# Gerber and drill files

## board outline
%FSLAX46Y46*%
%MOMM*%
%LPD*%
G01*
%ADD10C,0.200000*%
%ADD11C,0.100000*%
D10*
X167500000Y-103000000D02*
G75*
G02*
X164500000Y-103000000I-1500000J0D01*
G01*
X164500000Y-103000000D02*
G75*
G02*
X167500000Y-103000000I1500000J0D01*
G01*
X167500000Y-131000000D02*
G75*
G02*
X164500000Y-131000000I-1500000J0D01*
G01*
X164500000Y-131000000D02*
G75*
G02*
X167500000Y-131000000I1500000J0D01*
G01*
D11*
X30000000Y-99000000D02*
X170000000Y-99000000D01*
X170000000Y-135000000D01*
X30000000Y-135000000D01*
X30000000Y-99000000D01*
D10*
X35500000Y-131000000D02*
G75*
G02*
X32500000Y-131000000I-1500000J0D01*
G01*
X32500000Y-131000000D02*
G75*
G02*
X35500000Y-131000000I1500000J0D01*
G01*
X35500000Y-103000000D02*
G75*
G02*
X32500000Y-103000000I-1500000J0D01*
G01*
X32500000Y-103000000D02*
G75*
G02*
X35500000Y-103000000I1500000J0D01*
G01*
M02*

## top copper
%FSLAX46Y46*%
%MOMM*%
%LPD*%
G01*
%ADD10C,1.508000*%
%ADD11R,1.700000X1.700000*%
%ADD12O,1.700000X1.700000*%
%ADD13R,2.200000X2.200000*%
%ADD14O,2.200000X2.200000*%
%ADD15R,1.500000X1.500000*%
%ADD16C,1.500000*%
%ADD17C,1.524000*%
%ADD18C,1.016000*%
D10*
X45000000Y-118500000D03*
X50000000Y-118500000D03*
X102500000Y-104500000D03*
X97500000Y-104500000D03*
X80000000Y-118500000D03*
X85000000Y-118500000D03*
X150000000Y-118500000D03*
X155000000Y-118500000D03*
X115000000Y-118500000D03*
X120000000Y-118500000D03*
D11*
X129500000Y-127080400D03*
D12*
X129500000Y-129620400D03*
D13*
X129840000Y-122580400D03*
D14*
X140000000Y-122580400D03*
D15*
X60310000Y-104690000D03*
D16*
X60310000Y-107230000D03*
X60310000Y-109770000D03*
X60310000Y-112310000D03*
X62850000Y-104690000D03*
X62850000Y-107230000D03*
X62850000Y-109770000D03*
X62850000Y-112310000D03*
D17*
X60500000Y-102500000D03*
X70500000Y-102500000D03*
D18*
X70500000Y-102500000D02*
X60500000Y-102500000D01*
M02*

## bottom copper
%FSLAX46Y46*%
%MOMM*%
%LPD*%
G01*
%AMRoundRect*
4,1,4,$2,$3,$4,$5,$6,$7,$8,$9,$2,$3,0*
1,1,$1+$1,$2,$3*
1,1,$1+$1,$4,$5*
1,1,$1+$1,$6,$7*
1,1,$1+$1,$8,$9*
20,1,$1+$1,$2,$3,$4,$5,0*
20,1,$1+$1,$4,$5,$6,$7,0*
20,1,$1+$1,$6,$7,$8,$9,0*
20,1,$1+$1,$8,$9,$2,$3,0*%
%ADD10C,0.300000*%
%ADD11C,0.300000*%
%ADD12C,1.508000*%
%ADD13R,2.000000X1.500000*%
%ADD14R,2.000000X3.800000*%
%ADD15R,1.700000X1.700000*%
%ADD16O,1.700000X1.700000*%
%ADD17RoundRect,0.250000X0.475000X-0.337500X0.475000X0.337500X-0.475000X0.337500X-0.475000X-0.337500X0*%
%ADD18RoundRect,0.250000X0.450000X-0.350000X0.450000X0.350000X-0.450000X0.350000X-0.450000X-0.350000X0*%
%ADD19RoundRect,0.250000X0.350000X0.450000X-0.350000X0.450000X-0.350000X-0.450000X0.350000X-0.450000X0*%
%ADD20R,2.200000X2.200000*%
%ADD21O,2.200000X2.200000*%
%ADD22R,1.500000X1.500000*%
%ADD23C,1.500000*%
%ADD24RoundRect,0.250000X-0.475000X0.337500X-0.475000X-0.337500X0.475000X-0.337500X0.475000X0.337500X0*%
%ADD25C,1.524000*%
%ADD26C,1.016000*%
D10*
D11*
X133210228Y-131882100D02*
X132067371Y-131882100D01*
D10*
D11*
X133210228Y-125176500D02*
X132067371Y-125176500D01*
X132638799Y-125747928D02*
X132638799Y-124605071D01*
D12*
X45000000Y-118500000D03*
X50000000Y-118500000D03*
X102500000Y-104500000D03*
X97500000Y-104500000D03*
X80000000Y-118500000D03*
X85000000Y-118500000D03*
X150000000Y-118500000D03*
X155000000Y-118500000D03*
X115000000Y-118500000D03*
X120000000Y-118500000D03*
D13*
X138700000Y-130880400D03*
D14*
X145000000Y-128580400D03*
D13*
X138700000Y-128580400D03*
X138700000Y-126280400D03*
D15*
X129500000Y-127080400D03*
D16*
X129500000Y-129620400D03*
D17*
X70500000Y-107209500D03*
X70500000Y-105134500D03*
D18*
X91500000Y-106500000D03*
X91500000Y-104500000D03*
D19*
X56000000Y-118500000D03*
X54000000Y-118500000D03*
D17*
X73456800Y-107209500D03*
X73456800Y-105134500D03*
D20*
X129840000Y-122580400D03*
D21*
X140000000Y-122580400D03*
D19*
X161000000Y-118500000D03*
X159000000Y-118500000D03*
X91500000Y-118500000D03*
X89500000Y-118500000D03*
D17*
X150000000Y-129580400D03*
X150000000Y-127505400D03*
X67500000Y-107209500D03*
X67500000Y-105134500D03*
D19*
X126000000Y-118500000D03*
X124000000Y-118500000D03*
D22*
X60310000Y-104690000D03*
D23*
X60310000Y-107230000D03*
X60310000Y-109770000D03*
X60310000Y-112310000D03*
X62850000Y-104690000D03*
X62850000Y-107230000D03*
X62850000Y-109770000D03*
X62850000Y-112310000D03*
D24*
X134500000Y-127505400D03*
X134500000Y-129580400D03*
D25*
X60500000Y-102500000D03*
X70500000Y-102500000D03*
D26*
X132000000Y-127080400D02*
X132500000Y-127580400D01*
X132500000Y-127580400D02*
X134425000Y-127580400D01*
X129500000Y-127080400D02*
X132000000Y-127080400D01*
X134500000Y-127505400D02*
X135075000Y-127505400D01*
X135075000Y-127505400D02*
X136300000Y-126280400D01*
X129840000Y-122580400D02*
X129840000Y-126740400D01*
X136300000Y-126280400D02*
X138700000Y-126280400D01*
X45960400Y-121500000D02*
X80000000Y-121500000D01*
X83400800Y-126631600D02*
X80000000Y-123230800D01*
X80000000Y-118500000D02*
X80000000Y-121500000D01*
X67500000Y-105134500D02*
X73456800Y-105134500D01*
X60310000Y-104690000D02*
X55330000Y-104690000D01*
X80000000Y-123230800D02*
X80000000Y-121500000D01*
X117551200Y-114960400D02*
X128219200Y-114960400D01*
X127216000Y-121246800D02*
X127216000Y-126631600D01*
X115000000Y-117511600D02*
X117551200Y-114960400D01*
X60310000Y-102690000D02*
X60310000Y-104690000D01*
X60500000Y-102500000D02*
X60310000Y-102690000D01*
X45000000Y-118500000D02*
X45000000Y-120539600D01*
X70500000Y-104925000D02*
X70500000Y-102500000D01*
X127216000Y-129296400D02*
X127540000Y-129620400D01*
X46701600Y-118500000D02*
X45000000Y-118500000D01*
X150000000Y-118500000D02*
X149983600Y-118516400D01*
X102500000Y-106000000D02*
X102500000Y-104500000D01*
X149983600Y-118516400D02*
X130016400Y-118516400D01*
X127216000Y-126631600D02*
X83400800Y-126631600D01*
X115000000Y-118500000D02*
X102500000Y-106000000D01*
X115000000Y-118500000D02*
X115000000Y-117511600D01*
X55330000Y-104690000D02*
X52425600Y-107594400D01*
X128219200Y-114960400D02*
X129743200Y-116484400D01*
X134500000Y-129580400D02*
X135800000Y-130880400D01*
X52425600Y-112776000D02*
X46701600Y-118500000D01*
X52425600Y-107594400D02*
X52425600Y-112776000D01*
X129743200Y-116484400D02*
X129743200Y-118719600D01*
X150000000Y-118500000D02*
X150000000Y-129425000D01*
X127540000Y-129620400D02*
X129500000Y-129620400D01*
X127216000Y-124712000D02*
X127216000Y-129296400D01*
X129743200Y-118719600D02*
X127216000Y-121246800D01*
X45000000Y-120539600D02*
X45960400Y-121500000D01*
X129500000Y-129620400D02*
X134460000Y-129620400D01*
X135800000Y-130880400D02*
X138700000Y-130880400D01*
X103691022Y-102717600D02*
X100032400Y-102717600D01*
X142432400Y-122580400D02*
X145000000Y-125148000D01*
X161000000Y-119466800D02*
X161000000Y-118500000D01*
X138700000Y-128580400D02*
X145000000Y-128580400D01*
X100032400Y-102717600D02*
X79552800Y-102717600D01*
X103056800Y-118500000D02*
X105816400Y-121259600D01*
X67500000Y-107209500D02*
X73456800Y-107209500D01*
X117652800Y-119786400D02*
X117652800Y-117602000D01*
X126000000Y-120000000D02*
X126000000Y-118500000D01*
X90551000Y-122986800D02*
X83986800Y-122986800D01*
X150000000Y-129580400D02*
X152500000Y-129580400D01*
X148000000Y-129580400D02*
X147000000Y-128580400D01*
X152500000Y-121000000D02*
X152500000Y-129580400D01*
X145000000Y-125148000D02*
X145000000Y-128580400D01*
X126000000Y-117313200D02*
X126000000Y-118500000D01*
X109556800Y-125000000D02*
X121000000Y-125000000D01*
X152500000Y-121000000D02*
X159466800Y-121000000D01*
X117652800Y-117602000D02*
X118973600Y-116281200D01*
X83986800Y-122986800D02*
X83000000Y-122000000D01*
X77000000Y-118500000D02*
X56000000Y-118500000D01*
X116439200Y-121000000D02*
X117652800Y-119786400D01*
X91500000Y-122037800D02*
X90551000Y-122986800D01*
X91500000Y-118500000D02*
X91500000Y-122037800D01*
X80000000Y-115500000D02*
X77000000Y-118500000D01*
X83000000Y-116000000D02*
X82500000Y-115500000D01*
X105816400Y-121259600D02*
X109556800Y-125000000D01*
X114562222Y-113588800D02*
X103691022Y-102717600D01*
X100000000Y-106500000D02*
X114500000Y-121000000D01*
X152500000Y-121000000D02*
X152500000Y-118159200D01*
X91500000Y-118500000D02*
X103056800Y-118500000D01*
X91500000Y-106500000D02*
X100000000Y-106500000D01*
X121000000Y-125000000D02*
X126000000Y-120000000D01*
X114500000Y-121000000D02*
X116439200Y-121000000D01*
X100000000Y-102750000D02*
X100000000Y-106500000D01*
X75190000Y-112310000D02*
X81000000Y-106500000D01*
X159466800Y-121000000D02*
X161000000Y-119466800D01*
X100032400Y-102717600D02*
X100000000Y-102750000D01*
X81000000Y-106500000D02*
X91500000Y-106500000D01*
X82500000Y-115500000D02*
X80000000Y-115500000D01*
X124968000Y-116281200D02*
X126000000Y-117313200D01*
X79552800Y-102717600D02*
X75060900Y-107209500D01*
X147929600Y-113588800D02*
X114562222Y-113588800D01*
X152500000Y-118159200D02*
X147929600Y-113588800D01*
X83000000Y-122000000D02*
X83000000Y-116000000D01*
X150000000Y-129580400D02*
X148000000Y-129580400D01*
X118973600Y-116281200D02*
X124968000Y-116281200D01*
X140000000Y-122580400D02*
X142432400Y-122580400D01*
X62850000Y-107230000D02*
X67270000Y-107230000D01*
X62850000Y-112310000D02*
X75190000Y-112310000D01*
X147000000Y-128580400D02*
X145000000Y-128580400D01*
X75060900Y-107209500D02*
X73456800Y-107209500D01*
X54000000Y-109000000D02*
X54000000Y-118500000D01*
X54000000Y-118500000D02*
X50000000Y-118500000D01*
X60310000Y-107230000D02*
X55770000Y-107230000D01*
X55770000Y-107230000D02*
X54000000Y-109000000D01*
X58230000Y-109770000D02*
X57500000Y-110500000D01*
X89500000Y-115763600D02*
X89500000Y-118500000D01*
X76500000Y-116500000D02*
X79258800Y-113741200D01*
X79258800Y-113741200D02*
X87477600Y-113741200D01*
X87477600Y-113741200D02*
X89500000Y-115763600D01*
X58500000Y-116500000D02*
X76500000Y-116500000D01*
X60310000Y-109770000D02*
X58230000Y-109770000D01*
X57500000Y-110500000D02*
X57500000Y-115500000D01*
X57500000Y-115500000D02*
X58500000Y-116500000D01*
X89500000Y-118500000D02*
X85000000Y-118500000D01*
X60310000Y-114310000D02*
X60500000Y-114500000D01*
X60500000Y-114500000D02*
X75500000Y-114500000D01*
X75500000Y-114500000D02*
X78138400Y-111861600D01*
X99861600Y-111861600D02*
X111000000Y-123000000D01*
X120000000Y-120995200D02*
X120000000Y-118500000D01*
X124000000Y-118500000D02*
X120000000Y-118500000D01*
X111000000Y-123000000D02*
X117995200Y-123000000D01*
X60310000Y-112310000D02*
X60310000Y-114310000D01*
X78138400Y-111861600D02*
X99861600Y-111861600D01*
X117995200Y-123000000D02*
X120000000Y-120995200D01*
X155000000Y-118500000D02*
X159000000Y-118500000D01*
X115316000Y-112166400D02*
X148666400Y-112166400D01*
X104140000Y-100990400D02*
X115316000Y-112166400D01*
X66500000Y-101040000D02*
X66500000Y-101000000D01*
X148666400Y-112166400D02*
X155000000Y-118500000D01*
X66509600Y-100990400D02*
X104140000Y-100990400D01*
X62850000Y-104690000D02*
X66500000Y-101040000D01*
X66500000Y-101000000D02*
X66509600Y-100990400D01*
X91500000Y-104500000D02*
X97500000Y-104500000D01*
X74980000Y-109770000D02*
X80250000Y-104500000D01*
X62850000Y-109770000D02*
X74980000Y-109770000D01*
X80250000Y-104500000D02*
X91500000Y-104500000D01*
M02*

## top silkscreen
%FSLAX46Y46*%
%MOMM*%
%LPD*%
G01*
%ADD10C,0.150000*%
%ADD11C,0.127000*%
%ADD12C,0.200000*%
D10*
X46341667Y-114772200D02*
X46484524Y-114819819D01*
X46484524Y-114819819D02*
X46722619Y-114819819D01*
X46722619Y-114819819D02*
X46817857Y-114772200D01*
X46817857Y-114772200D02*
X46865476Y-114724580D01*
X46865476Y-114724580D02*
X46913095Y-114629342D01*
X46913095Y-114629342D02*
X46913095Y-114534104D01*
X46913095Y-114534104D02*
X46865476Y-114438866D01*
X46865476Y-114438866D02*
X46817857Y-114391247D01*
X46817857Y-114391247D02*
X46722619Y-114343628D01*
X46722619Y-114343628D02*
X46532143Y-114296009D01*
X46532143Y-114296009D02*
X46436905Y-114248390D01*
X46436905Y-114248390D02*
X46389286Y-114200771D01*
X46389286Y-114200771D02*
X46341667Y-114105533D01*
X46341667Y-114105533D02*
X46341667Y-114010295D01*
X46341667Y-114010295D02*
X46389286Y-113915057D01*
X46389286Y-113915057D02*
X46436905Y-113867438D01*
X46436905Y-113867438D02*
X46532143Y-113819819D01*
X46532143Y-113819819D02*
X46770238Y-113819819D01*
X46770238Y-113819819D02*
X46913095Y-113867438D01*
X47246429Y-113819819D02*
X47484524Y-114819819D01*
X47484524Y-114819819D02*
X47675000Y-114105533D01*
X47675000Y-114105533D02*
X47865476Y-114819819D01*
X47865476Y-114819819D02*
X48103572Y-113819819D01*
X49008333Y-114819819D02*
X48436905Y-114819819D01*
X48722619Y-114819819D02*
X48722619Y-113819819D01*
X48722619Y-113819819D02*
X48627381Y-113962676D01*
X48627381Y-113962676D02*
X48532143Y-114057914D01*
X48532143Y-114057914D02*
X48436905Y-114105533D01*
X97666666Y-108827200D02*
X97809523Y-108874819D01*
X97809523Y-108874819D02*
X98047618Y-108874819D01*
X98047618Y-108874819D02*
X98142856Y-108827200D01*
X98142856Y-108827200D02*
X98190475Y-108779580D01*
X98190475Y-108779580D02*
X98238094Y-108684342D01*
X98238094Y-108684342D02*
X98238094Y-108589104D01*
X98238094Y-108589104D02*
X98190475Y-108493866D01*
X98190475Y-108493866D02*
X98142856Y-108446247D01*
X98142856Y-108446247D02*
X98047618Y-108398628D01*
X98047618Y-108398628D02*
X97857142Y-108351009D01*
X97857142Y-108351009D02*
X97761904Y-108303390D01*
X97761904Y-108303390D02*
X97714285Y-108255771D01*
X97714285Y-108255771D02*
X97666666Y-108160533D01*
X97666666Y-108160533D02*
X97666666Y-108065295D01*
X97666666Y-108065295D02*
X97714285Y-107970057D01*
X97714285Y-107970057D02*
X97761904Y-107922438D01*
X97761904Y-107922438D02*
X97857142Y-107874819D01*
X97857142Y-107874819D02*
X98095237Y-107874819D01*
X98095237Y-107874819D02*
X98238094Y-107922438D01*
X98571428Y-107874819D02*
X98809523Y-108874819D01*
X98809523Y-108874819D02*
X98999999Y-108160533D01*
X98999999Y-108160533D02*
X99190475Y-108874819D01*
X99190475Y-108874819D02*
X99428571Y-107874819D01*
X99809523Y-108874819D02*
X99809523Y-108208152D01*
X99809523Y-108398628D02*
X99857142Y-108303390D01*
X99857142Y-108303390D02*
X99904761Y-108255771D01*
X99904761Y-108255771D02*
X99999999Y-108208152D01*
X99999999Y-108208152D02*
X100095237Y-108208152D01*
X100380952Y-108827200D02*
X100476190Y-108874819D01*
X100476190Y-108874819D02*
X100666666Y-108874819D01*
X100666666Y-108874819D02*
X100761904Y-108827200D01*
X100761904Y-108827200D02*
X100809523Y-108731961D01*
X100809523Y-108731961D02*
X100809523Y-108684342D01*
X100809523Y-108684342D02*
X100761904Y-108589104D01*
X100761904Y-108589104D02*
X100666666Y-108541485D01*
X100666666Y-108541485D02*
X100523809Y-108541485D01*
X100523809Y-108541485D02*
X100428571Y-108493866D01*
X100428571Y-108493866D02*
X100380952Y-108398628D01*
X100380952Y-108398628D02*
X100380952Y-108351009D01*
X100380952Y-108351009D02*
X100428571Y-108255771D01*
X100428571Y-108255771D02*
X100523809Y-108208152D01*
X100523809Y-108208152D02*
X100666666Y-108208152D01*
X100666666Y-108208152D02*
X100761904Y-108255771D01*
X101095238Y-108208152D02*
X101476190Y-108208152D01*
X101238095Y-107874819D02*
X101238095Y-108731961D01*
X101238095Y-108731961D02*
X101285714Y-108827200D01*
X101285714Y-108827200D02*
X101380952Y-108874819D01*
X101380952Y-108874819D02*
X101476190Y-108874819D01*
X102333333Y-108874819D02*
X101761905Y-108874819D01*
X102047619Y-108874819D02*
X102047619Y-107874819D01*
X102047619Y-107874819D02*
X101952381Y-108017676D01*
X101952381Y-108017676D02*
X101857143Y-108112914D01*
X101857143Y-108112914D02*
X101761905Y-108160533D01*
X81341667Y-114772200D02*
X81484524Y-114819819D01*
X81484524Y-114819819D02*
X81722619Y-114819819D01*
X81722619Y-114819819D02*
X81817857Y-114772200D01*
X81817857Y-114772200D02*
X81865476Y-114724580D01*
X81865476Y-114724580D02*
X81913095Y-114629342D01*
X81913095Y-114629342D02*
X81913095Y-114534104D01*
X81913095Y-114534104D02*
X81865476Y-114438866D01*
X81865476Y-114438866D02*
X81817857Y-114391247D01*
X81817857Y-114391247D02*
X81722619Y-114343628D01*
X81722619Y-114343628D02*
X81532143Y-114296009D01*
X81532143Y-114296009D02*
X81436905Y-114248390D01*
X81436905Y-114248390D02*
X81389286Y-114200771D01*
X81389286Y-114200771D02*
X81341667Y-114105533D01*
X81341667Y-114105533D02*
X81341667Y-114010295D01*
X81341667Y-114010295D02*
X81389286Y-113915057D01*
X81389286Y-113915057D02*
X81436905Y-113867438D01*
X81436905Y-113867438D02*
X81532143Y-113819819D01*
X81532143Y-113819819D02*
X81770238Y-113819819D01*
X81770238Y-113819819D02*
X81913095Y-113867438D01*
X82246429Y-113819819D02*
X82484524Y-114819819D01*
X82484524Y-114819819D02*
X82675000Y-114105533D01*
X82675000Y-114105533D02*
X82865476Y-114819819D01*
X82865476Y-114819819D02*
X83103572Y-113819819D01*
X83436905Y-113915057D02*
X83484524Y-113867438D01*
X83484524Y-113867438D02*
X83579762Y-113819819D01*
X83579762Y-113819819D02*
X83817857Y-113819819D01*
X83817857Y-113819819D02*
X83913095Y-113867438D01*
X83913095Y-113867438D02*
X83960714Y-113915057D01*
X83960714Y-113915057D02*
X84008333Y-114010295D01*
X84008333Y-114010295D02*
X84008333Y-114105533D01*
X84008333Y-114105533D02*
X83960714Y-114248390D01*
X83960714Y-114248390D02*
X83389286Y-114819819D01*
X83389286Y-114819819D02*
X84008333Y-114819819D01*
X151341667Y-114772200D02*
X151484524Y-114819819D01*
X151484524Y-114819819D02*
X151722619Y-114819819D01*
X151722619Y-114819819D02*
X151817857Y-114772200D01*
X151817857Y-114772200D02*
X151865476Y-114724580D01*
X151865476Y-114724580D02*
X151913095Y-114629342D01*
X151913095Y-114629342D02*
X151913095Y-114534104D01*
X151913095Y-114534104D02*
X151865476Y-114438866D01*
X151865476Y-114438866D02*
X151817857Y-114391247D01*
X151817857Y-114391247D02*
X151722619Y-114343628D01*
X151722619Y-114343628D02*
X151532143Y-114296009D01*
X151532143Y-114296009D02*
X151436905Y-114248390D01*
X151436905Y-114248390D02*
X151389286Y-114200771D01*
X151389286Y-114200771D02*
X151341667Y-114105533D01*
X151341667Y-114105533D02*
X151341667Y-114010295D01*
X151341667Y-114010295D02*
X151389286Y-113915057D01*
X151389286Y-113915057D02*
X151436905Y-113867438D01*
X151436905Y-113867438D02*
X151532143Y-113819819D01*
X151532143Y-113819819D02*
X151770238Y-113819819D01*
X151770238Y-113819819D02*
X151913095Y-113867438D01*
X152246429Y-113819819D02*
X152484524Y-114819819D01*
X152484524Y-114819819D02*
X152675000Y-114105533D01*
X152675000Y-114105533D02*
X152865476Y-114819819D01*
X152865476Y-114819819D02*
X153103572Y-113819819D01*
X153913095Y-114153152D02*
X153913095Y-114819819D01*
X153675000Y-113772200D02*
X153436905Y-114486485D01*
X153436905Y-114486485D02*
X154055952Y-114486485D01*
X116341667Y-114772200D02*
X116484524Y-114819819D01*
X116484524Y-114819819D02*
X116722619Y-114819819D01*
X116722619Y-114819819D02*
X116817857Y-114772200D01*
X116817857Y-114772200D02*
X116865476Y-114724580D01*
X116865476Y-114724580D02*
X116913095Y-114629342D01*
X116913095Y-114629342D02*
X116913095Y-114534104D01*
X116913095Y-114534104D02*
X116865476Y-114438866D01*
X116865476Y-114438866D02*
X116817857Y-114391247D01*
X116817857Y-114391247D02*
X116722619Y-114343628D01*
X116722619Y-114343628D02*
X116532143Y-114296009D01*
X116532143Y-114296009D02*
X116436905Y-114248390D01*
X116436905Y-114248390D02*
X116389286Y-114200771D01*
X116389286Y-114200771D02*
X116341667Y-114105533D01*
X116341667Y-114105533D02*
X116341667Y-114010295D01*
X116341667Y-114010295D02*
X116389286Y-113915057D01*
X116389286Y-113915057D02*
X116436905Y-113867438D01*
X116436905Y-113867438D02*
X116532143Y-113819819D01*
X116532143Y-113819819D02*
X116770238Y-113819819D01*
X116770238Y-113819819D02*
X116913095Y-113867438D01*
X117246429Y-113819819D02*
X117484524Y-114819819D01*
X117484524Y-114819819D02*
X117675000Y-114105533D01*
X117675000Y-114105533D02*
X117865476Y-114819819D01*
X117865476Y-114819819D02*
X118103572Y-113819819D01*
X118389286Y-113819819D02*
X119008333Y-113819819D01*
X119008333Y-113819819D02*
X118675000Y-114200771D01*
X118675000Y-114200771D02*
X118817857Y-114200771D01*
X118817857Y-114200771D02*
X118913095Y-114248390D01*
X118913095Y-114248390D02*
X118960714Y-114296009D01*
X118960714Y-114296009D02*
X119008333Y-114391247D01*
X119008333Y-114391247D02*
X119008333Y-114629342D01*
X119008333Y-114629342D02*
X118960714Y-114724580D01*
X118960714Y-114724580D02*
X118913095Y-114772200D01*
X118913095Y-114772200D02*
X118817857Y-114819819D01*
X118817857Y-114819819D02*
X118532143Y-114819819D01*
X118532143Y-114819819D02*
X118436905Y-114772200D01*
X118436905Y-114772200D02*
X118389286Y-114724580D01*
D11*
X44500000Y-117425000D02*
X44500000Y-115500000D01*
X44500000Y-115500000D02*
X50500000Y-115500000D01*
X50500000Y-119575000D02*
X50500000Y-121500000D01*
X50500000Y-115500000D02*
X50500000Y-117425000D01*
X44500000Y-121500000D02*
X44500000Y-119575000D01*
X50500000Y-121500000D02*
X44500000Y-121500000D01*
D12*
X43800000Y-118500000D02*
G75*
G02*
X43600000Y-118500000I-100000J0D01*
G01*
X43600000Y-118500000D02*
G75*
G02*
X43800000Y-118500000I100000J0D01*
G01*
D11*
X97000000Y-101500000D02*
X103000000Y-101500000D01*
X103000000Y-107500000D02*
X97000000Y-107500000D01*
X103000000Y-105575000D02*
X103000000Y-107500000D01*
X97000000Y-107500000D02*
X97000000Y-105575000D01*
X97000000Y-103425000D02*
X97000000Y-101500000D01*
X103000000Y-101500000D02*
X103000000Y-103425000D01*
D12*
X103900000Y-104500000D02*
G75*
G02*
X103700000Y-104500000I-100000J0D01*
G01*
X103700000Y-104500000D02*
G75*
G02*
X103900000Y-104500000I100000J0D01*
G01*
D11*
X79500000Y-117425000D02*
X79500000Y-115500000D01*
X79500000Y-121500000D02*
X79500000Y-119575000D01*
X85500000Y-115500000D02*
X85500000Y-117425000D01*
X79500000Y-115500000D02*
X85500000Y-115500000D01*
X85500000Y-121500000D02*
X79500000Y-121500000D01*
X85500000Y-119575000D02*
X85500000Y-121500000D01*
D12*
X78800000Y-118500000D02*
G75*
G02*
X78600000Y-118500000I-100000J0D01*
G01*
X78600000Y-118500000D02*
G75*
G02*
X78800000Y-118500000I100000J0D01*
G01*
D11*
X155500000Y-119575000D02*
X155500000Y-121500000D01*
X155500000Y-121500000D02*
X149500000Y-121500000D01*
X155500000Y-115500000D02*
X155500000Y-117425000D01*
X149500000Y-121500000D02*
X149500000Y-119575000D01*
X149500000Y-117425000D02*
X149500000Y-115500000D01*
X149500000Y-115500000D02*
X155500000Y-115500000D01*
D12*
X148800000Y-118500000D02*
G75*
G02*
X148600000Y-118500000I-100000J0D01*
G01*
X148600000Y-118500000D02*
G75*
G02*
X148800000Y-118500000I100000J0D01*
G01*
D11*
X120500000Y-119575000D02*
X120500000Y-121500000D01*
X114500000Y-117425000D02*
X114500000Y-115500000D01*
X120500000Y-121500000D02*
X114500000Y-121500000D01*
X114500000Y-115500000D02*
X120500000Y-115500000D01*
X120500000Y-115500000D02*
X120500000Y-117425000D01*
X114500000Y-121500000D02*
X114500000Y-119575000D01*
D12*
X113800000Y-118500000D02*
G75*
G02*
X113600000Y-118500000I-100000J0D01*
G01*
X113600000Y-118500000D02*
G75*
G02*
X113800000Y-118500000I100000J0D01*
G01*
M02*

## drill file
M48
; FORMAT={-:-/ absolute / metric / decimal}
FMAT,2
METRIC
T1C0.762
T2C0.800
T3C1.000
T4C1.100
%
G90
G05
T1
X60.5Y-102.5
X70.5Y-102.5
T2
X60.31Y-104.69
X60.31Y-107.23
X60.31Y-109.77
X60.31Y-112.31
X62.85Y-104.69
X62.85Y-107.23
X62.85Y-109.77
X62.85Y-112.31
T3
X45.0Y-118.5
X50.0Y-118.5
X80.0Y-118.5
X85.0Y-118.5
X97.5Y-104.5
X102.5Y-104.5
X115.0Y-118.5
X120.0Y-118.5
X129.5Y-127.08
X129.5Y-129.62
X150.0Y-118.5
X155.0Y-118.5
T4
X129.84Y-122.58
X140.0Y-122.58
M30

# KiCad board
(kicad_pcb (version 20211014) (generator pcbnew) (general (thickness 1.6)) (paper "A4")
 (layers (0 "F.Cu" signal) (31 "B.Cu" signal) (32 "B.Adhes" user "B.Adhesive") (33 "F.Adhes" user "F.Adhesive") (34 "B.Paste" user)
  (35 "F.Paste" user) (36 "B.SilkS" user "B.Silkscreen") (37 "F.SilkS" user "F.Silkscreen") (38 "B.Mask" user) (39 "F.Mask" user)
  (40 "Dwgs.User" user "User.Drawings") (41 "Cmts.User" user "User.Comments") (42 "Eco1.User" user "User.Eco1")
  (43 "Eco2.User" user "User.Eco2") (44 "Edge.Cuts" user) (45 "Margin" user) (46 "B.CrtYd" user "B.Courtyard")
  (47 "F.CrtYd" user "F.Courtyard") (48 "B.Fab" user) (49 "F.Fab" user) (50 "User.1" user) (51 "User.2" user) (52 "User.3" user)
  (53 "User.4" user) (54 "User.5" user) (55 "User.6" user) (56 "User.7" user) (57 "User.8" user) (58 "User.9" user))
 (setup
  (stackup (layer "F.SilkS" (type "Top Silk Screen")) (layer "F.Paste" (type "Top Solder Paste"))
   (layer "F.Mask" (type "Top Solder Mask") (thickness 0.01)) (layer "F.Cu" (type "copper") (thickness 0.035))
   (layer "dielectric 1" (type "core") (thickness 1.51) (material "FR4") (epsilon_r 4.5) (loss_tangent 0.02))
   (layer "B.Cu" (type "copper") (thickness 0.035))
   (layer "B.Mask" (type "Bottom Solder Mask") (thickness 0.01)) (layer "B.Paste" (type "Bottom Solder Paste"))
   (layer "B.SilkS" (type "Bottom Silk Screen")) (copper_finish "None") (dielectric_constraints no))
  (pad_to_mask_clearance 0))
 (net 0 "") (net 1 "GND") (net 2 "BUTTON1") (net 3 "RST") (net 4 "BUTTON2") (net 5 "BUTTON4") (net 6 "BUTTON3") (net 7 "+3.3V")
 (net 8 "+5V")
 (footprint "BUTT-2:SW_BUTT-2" (layer "F.Cu") (at 47.5 118.5)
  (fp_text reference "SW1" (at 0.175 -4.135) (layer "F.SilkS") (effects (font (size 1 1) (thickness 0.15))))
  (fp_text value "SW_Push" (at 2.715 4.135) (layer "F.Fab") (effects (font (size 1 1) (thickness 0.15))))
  (fp_line (start -3 -1.075) (end -3 -3) (layer "F.SilkS") (width 0.127))
  (fp_line (start -3 -3) (end 3 -3) (layer "F.SilkS") (width 0.127))
  (fp_line (start 3 1.075) (end 3 3) (layer "F.SilkS") (width 0.127))
  (fp_line (start 3 -3) (end 3 -1.075) (layer "F.SilkS") (width 0.127))
  (fp_line (start -3 3) (end -3 1.075) (layer "F.SilkS") (width 0.127))
  (fp_line (start 3 3) (end -3 3) (layer "F.SilkS") (width 0.127))
  (fp_circle (center -3.8 0) (end -3.7 0) (layer "F.SilkS") (width 0.2) (fill none))
  (pad "1" thru_hole circle locked (at -2.5 0) (size 1.508 1.508) (drill 1) (layers *.Cu *.Mask) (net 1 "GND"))
  (pad "2" thru_hole circle locked (at 2.5 0) (size 1.508 1.508) (drill 1) (layers *.Cu *.Mask) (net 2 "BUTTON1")))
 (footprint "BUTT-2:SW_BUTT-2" (layer "F.Cu") (at 100 104.5 180)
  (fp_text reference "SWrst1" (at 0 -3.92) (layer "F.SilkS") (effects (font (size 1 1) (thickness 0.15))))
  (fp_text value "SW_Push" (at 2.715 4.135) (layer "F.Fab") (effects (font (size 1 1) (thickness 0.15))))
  (fp_line (start 3 3) (end -3 3) (layer "F.SilkS") (width 0.127))
  (fp_line (start -3 -3) (end 3 -3) (layer "F.SilkS") (width 0.127))
  (fp_line (start -3 -1.075) (end -3 -3) (layer "F.SilkS") (width 0.127))
  (fp_line (start 3 -3) (end 3 -1.075) (layer "F.SilkS") (width 0.127))
  (fp_line (start 3 1.075) (end 3 3) (layer "F.SilkS") (width 0.127))
  (fp_line (start -3 3) (end -3 1.075) (layer "F.SilkS") (width 0.127))
  (fp_circle (center -3.8 0) (end -3.7 0) (layer "F.SilkS") (width 0.2) (fill none))
  (pad "1" thru_hole circle locked (at -2.5 0 180) (size 1.508 1.508) (drill 1) (layers *.Cu *.Mask) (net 1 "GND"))
  (pad "2" thru_hole circle locked (at 2.5 0 180) (size 1.508 1.508) (drill 1) (layers *.Cu *.Mask) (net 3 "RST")))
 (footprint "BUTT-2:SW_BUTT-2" (layer "F.Cu") (at 82.5 118.5)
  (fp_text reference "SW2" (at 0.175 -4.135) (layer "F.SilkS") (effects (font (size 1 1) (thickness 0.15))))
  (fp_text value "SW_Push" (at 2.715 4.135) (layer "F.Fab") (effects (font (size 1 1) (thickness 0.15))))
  (fp_line (start -3 -1.075) (end -3 -3) (layer "F.SilkS") (width 0.127))
  (fp_line (start -3 3) (end -3 1.075) (layer "F.SilkS") (width 0.127))
  (fp_line (start 3 -3) (end 3 -1.075) (layer "F.SilkS") (width 0.127))
  (fp_line (start -3 -3) (end 3 -3) (layer "F.SilkS") (width 0.127))
  (fp_line (start 3 3) (end -3 3) (layer "F.SilkS") (width 0.127))
  (fp_line (start 3 1.075) (end 3 3) (layer "F.SilkS") (width 0.127))
  (fp_circle (center -3.8 0) (end -3.7 0) (layer "F.SilkS") (width 0.2) (fill none))
  (pad "1" thru_hole circle locked (at -2.5 0) (size 1.508 1.508) (drill 1) (layers *.Cu *.Mask) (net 1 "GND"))
  (pad "2" thru_hole circle locked (at 2.5 0) (size 1.508 1.508) (drill 1) (layers *.Cu *.Mask) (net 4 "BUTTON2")))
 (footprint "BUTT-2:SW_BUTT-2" (layer "F.Cu") (at 152.5 118.5)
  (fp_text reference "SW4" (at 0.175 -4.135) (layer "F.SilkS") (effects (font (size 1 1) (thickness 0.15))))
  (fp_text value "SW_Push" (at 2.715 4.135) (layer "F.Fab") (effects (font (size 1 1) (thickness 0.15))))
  (fp_line (start 3 1.075) (end 3 3) (layer "F.SilkS") (width 0.127))
  (fp_line (start 3 3) (end -3 3) (layer "F.SilkS") (width 0.127))
  (fp_line (start 3 -3) (end 3 -1.075) (layer "F.SilkS") (width 0.127))
  (fp_line (start -3 3) (end -3 1.075) (layer "F.SilkS") (width 0.127))
  (fp_line (start -3 -1.075) (end -3 -3) (layer "F.SilkS") (width 0.127))
  (fp_line (start -3 -3) (end 3 -3) (layer "F.SilkS") (width 0.127))
  (fp_circle (center -3.8 0) (end -3.7 0) (layer "F.SilkS") (width 0.2) (fill none))
  (pad "1" thru_hole circle locked (at -2.5 0) (size 1.508 1.508) (drill 1) (layers *.Cu *.Mask) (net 1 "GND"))
  (pad "2" thru_hole circle locked (at 2.5 0) (size 1.508 1.508) (drill 1) (layers *.Cu *.Mask) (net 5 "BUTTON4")))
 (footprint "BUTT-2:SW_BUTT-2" (layer "F.Cu") (at 117.5 118.5)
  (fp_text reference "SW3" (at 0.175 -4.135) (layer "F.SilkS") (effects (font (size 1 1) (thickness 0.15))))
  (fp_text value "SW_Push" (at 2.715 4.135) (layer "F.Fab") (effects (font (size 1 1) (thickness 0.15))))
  (fp_line (start 3 1.075) (end 3 3) (layer "F.SilkS") (width 0.127))
  (fp_line (start -3 -1.075) (end -3 -3) (layer "F.SilkS") (width 0.127))
  (fp_line (start 3 3) (end -3 3) (layer "F.SilkS") (width 0.127))
  (fp_line (start -3 -3) (end 3 -3) (layer "F.SilkS") (width 0.127))
  (fp_line (start 3 -3) (end 3 -1.075) (layer "F.SilkS") (width 0.127))
  (fp_line (start -3 3) (end -3 1.075) (layer "F.SilkS") (width 0.127))
  (fp_circle (center -3.8 0) (end -3.7 0) (layer "F.SilkS") (width 0.2) (fill none))
  (pad "1" thru_hole circle locked (at -2.5 0) (size 1.508 1.508) (drill 1) (layers *.Cu *.Mask) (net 1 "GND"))
  (pad "2" thru_hole circle locked (at 2.5 0) (size 1.508 1.508) (drill 1) (layers *.Cu *.Mask) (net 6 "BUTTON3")))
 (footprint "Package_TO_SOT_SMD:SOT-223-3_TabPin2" (layer "B.Cu") (at 141.85 128.5804)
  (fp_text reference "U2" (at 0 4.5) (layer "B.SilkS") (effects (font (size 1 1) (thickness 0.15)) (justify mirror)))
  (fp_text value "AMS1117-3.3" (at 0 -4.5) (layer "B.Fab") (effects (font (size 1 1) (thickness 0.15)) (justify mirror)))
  (pad "1" smd rect (at -3.15 2.3) (size 2 1.5) (layers "B.Cu" "B.Paste" "B.Mask") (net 1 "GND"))
  (pad "2" smd rect (at 3.15 0) (size 2 3.8) (layers "B.Cu" "B.Paste" "B.Mask") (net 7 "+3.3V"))
  (pad "2" smd rect (at -3.15 0) (size 2 1.5) (layers "B.Cu" "B.Paste" "B.Mask") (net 7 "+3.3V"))
  (pad "3" smd rect (at -3.15 -2.3) (size 2 1.5) (layers "B.Cu" "B.Paste" "B.Mask") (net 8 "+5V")))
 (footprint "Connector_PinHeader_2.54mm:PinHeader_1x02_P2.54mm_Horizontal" (layer "B.Cu") (at 129.5 127.0804 180)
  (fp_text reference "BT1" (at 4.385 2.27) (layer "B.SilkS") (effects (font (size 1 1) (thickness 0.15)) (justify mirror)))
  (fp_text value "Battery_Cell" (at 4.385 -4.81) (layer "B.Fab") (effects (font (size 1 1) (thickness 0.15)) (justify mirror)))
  (pad "1" thru_hole rect (at 0 0 180) (size 1.7 1.7) (drill 1) (layers *.Cu *.Mask) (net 8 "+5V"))
  (pad "2" thru_hole oval (at 0 -2.54 180) (size 1.7 1.7) (drill 1) (layers *.Cu *.Mask) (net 1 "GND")))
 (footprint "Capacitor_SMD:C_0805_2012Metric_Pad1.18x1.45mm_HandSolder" (layer "B.Cu") (at 70.5 106.172 90)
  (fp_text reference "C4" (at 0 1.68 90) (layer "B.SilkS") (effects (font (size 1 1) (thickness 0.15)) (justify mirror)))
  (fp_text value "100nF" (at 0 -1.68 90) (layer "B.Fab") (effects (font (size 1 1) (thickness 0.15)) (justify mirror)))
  (pad "1" smd roundrect (at -1.0375 0 90) (size 1.175 1.45) (layers "B.Cu" "B.Paste" "B.Mask") (roundrect_rratio 0.2127659574)
   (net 7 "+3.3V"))
  (pad "2" smd roundrect (at 1.0375 0 90) (size 1.175 1.45) (layers "B.Cu" "B.Paste" "B.Mask") (roundrect_rratio 0.2127659574) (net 1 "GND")))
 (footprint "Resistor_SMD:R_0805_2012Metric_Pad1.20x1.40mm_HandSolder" (layer "B.Cu") (at 91.5 105.5 90)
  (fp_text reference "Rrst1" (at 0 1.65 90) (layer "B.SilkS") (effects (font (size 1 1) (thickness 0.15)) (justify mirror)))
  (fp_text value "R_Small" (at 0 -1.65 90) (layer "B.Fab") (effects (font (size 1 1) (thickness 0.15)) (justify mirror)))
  (pad "1" smd roundrect (at -1 0 90) (size 1.2 1.4) (layers "B.Cu" "B.Paste" "B.Mask") (roundrect_rratio 0.2083333333) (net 7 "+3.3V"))
  (pad "2" smd roundrect (at 1 0 90) (size 1.2 1.4) (layers "B.Cu" "B.Paste" "B.Mask") (roundrect_rratio 0.2083333333) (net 3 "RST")))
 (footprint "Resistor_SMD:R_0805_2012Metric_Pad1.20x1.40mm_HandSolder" (layer "B.Cu") (at 55 118.5 180)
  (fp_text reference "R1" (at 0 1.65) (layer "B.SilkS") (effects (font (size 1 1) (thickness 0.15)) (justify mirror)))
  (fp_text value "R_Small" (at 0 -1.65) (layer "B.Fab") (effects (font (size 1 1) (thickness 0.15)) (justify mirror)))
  (pad "1" smd roundrect (at -1 0 180) (size 1.2 1.4) (layers "B.Cu" "B.Paste" "B.Mask") (roundrect_rratio 0.2083333333) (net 7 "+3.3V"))
  (pad "2" smd roundrect (at 1 0 180) (size 1.2 1.4) (layers "B.Cu" "B.Paste" "B.Mask") (roundrect_rratio 0.2083333333) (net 2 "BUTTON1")))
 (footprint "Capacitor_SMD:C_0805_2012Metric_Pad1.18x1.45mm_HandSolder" (layer "B.Cu") (at 73.4568 106.172 90)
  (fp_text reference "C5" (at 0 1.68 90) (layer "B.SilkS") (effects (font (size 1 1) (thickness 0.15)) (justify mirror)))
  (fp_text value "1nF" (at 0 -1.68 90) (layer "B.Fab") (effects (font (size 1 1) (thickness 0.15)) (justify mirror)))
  (pad "1" smd roundrect (at -1.0375 0 90) (size 1.175 1.45) (layers "B.Cu" "B.Paste" "B.Mask") (roundrect_rratio 0.2127659574)
   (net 7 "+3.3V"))
  (pad "2" smd roundrect (at 1.0375 0 90) (size 1.175 1.45) (layers "B.Cu" "B.Paste" "B.Mask") (roundrect_rratio 0.2127659574) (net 1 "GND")))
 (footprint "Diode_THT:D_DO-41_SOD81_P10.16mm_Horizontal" (layer "B.Cu") (at 129.84 122.5804)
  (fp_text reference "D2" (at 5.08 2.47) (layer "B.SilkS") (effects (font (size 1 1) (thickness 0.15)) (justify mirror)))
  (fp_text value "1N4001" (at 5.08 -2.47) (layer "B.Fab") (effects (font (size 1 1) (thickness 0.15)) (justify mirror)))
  (pad "1" thru_hole rect (at 0 0) (size 2.2 2.2) (drill 1.1) (layers *.Cu *.Mask) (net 8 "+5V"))
  (pad "2" thru_hole oval (at 10.16 0) (size 2.2 2.2) (drill 1.1) (layers *.Cu *.Mask) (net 7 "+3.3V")))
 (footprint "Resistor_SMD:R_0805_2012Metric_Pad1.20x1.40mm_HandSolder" (layer "B.Cu") (at 160 118.5 180)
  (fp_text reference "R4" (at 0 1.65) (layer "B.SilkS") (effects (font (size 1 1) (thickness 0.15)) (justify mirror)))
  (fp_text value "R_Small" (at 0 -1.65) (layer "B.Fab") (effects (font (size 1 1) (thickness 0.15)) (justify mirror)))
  (pad "1" smd roundrect (at -1 0 180) (size 1.2 1.4) (layers "B.Cu" "B.Paste" "B.Mask") (roundrect_rratio 0.2083333333) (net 7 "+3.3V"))
  (pad "2" smd roundrect (at 1 0 180) (size 1.2 1.4) (layers "B.Cu" "B.Paste" "B.Mask") (roundrect_rratio 0.2083333333) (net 5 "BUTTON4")))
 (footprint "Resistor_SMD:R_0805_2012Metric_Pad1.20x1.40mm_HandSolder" (layer "B.Cu") (at 90.5 118.5 180)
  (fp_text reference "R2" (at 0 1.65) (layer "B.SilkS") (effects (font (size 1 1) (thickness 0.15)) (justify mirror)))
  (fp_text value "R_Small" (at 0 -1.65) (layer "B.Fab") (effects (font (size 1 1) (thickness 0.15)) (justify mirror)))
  (pad "1" smd roundrect (at -1 0 180) (size 1.2 1.4) (layers "B.Cu" "B.Paste" "B.Mask") (roundrect_rratio 0.2083333333) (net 7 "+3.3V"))
  (pad "2" smd roundrect (at 1 0 180) (size 1.2 1.4) (layers "B.Cu" "B.Paste" "B.Mask") (roundrect_rratio 0.2083333333) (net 4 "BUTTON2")))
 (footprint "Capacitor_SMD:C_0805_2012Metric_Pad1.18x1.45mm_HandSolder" (layer "B.Cu") (at 150 128.5429 90)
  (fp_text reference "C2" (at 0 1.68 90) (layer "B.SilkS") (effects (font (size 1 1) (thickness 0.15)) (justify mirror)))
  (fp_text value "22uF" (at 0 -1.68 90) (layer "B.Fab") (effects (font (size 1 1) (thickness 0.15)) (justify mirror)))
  (pad "1" smd roundrect (at -1.0375 0 90) (size 1.175 1.45) (layers "B.Cu" "B.Paste" "B.Mask") (roundrect_rratio 0.2127659574)
   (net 7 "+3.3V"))
  (pad "2" smd roundrect (at 1.0375 0 90) (size 1.175 1.45) (layers "B.Cu" "B.Paste" "B.Mask") (roundrect_rratio 0.2127659574) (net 1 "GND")))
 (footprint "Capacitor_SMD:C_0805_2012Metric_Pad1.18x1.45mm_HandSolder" (layer "B.Cu") (at 67.5 106.172 90)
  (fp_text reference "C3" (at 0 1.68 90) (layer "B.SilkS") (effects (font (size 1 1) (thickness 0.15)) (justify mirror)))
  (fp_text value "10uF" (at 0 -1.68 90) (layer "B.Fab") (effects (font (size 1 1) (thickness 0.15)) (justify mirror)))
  (pad "1" smd roundrect (at -1.0375 0 90) (size 1.175 1.45) (layers "B.Cu" "B.Paste" "B.Mask") (roundrect_rratio 0.2127659574)
   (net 7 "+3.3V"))
  (pad "2" smd roundrect (at 1.0375 0 90) (size 1.175 1.45) (layers "B.Cu" "B.Paste" "B.Mask") (roundrect_rratio 0.2127659574) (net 1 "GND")))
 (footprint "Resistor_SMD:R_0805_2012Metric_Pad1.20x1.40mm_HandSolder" (layer "B.Cu") (at 125 118.5 180)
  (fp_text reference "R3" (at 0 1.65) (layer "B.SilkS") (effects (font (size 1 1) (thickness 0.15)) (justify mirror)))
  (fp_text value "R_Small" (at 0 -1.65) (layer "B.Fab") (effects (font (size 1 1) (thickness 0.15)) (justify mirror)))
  (pad "1" smd roundrect (at -1 0 180) (size 1.2 1.4) (layers "B.Cu" "B.Paste" "B.Mask") (roundrect_rratio 0.2083333333) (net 7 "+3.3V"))
  (pad "2" smd roundrect (at 1 0 180) (size 1.2 1.4) (layers "B.Cu" "B.Paste" "B.Mask") (roundrect_rratio 0.2083333333) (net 6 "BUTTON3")))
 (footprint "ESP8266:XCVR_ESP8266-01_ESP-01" (layer "B.Cu") (at 52 108.5 -90)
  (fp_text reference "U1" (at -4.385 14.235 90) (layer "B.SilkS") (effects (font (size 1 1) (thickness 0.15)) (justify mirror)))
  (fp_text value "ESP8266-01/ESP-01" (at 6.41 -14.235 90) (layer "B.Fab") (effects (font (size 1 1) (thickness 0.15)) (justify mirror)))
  (pad "1" thru_hole rect (at -3.81 -8.31 270) (size 1.5 1.5) (drill 0.8) (layers *.Cu *.Mask) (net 1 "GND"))
  (pad "2" thru_hole circle (at -1.27 -8.31 270) (size 1.5 1.5) (drill 0.8) (layers *.Cu *.Mask) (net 2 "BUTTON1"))
  (pad "3" thru_hole circle (at 1.27 -8.31 270) (size 1.5 1.5) (drill 0.8) (layers *.Cu *.Mask) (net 4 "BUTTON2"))
  (pad "4" thru_hole circle (at 3.81 -8.31 270) (size 1.5 1.5) (drill 0.8) (layers *.Cu *.Mask) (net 6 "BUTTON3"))
  (pad "5" thru_hole circle (at -3.81 -10.85 270) (size 1.5 1.5) (drill 0.8) (layers *.Cu *.Mask) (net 5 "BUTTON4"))
  (pad "6" thru_hole circle (at -1.27 -10.85 270) (size 1.5 1.5) (drill 0.8) (layers *.Cu *.Mask) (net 7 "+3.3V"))
  (pad "7" thru_hole circle (at 1.27 -10.85 270) (size 1.5 1.5) (drill 0.8) (layers *.Cu *.Mask) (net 3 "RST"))
  (pad "8" thru_hole circle (at 3.81 -10.85 270) (size 1.5 1.5) (drill 0.8) (layers *.Cu *.Mask) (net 7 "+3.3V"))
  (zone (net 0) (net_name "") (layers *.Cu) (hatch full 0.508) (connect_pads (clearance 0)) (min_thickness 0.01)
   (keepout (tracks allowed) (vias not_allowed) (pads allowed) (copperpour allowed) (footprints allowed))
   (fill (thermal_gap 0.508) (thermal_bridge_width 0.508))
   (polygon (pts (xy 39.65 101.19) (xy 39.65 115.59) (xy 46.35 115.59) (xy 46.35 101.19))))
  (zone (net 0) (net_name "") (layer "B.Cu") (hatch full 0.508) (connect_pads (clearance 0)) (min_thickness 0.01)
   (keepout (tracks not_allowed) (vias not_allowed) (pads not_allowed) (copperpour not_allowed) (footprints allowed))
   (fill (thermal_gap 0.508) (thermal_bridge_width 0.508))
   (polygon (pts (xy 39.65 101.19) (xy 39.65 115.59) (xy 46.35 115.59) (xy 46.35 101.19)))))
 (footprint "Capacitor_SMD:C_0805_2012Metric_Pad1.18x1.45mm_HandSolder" (layer "B.Cu") (at 134.5 128.5429 -90)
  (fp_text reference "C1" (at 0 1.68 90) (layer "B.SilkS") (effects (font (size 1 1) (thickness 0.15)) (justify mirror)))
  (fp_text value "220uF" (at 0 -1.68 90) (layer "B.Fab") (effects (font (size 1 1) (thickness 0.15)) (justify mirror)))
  (pad "1" smd roundrect (at -1.0375 0 270) (size 1.175 1.45) (layers "B.Cu" "B.Paste" "B.Mask") (roundrect_rratio 0.2127659574)
   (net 8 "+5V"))
  (pad "2" smd roundrect (at 1.0375 0 270) (size 1.175 1.45) (layers "B.Cu" "B.Paste" "B.Mask") (roundrect_rratio 0.2127659574)
   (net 1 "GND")))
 (gr_circle (center 166 103) (end 167.5 103) (layer "Edge.Cuts") (width 0.2) (fill none))
 (gr_circle (center 166 131) (end 167.5 131) (layer "Edge.Cuts") (width 0.2) (fill none))
 (gr_rect (start 30 99) (end 170 135) (layer "Edge.Cuts") (width 0.1) (fill none))
 (gr_circle (center 34 131) (end 35.5 131) (layer "Edge.Cuts") (width 0.2) (fill none))
 (gr_circle (center 34 103) (end 35.5 103) (layer "Edge.Cuts") (width 0.2) (fill none))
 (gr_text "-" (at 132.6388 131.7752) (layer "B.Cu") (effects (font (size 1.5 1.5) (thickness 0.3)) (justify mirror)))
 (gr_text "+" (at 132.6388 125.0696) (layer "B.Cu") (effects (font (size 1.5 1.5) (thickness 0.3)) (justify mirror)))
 (segment (start 132 127.0804) (end 132.5 127.5804) (width 1.016) (layer "B.Cu") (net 8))
 (segment (start 132.5 127.5804) (end 134.425 127.5804) (width 1.016) (layer "B.Cu") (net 8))
 (segment (start 129.5 127.0804) (end 132 127.0804) (width 1.016) (layer "B.Cu") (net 8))
 (segment (start 134.5 127.5054) (end 135.075 127.5054) (width 1.016) (layer "B.Cu") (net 8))
 (segment (start 135.075 127.5054) (end 136.3 126.2804) (width 1.016) (layer "B.Cu") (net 8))
 (segment (start 129.84 122.5804) (end 129.84 126.7404) (width 1.016) (layer "B.Cu") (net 8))
 (segment (start 136.3 126.2804) (end 138.7 126.2804) (width 1.016) (layer "B.Cu") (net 8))
 (segment (start 70.5 102.5) (end 60.5 102.5) (width 1.016) (layer "F.Cu") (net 1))
 (via (at 60.5 102.5) (size 1.524) (drill 0.762) (layers "F.Cu" "B.Cu") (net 1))
 (via (at 70.5 102.5) (size 1.524) (drill 0.762) (layers "F.Cu" "B.Cu") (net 1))
 (segment (start 45.9604 121.5) (end 80 121.5) (width 1.016) (layer "B.Cu") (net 1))
 (segment (start 83.4008 126.6316) (end 80 123.2308) (width 1.016) (layer "B.Cu") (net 1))
 (segment (start 80 118.5) (end 80 121.5) (width 1.016) (layer "B.Cu") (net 1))
 (segment (start 67.5 105.1345) (end 73.4568 105.1345) (width 1.016) (layer "B.Cu") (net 1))
 (segment (start 60.31 104.69) (end 55.33 104.69) (width 1.016) (layer "B.Cu") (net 1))
 (segment (start 80 123.2308) (end 80 121.5) (width 1.016) (layer "B.Cu") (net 1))
 (segment (start 117.5512 114.9604) (end 128.2192 114.9604) (width 1.016) (layer "B.Cu") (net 1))
 (segment (start 127.216 121.2468) (end 127.216 126.6316) (width 1.016) (layer "B.Cu") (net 1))
 (segment (start 115 117.5116) (end 117.5512 114.9604) (width 1.016) (layer "B.Cu") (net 1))
 (segment (start 60.31 102.69) (end 60.31 104.69) (width 1.016) (layer "B.Cu") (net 1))
 (segment (start 60.5 102.5) (end 60.31 102.69) (width 1.016) (layer "B.Cu") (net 1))
 (segment (start 45 118.5) (end 45 120.5396) (width 1.016) (layer "B.Cu") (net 1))
 (segment (start 70.5 104.925) (end 70.5 102.5) (width 1.016) (layer "B.Cu") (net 1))
 (segment (start 127.216 129.2964) (end 127.54 129.6204) (width 1.016) (layer "B.Cu") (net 1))
 (segment (start 46.7016 118.5) (end 45 118.5) (width 1.016) (layer "B.Cu") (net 1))
 (segment (start 150 118.5) (end 149.9836 118.5164) (width 1.016) (layer "B.Cu") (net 1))
 (segment (start 102.5 106) (end 102.5 104.5) (width 1.016) (layer "B.Cu") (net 1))
 (segment (start 149.9836 118.5164) (end 130.0164 118.5164) (width 1.016) (layer "B.Cu") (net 1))
 (segment (start 127.216 126.6316) (end 83.4008 126.6316) (width 1.016) (layer "B.Cu") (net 1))
 (segment (start 115 118.5) (end 102.5 106) (width 1.016) (layer "B.Cu") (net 1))
 (segment (start 115 118.5) (end 115 117.5116) (width 1.016) (layer "B.Cu") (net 1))
 (segment (start 55.33 104.69) (end 52.4256 107.5944) (width 1.016) (layer "B.Cu") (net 1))
 (segment (start 128.2192 114.9604) (end 129.7432 116.4844) (width 1.016) (layer "B.Cu") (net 1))
 (segment (start 134.5 129.5804) (end 135.8 130.8804) (width 1.016) (layer "B.Cu") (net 1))
 (segment (start 52.4256 112.776) (end 46.7016 118.5) (width 1.016) (layer "B.Cu") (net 1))
 (segment (start 52.4256 107.5944) (end 52.4256 112.776) (width 1.016) (layer "B.Cu") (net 1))
 (segment (start 129.7432 116.4844) (end 129.7432 118.7196) (width 1.016) (layer "B.Cu") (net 1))
 (segment (start 150 118.5) (end 150 129.425) (width 1.016) (layer "B.Cu") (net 1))
 (segment (start 127.54 129.6204) (end 129.5 129.6204) (width 1.016) (layer "B.Cu") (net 1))
 (segment (start 127.216 124.712) (end 127.216 129.2964) (width 1.016) (layer "B.Cu") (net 1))
 (segment (start 129.7432 118.7196) (end 127.216 121.2468) (width 1.016) (layer "B.Cu") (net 1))
 (segment (start 45 120.5396) (end 45.9604 121.5) (width 1.016) (layer "B.Cu") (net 1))
 (segment (start 129.5 129.6204) (end 134.46 129.6204) (width 1.016) (layer "B.Cu") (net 1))
 (segment (start 135.8 130.8804) (end 138.7 130.8804) (width 1.016) (layer "B.Cu") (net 1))
 (segment (start 103.691022 102.7176) (end 100.0324 102.7176) (width 1.016) (layer "B.Cu") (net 7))
 (segment (start 142.4324 122.5804) (end 145 125.148) (width 1.016) (layer "B.Cu") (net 7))
 (segment (start 161 119.4668) (end 161 118.5) (width 1.016) (layer "B.Cu") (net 7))
 (segment (start 138.7 128.5804) (end 145 128.5804) (width 1.016) (layer "B.Cu") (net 7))
 (segment (start 100.0324 102.7176) (end 79.5528 102.7176) (width 1.016) (layer "B.Cu") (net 7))
 (segment (start 103.0568 118.5) (end 105.8164 121.2596) (width 1.016) (layer "B.Cu") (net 7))
 (segment (start 67.5 107.2095) (end 73.4568 107.2095) (width 1.016) (layer "B.Cu") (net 7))
 (segment (start 117.6528 119.7864) (end 117.6528 117.602) (width 1.016) (layer "B.Cu") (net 7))
 (segment (start 126 120) (end 126 118.5) (width 1.016) (layer "B.Cu") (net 7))
 (segment (start 90.551 122.9868) (end 83.9868 122.9868) (width 1.016) (layer "B.Cu") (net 7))
 (segment (start 150 129.5804) (end 152.5 129.5804) (width 1.016) (layer "B.Cu") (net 7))
 (segment (start 148 129.5804) (end 147 128.5804) (width 1.016) (layer "B.Cu") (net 7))
 (segment (start 152.5 121) (end 152.5 129.5804) (width 1.016) (layer "B.Cu") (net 7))
 (segment (start 145 125.148) (end 145 128.5804) (width 1.016) (layer "B.Cu") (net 7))
 (segment (start 126 117.3132) (end 126 118.5) (width 1.016) (layer "B.Cu") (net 7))
 (segment (start 109.5568 125) (end 121 125) (width 1.016) (layer "B.Cu") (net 7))
 (segment (start 152.5 121) (end 159.4668 121) (width 1.016) (layer "B.Cu") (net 7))
 (segment (start 117.6528 117.602) (end 118.9736 116.2812) (width 1.016) (layer "B.Cu") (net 7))
 (segment (start 83.9868 122.9868) (end 83 122) (width 1.016) (layer "B.Cu") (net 7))
 (segment (start 77 118.5) (end 56 118.5) (width 1.016) (layer "B.Cu") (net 7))
 (segment (start 116.4392 121) (end 117.6528 119.7864) (width 1.016) (layer "B.Cu") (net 7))
 (segment (start 91.5 122.0378) (end 90.551 122.9868) (width 1.016) (layer "B.Cu") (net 7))
 (segment (start 91.5 118.5) (end 91.5 122.0378) (width 1.016) (layer "B.Cu") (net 7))
 (segment (start 80 115.5) (end 77 118.5) (width 1.016) (layer "B.Cu") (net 7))
 (segment (start 83 116) (end 82.5 115.5) (width 1.016) (layer "B.Cu") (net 7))
 (segment (start 105.8164 121.2596) (end 109.5568 125) (width 1.016) (layer "B.Cu") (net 7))
 (segment (start 114.562222 113.5888) (end 103.691022 102.7176) (width 1.016) (layer "B.Cu") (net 7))
 (segment (start 100 106.5) (end 114.5 121) (width 1.016) (layer "B.Cu") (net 7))
 (segment (start 152.5 121) (end 152.5 118.1592) (width 1.016) (layer "B.Cu") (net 7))
 (segment (start 91.5 118.5) (end 103.0568 118.5) (width 1.016) (layer "B.Cu") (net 7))
 (segment (start 91.5 106.5) (end 100 106.5) (width 1.016) (layer "B.Cu") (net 7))
 (segment (start 121 125) (end 126 120) (width 1.016) (layer "B.Cu") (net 7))
 (segment (start 114.5 121) (end 116.4392 121) (width 1.016) (layer "B.Cu") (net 7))
 (segment (start 100 102.75) (end 100 106.5) (width 1.016) (layer "B.Cu") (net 7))
 (segment (start 75.19 112.31) (end 81 106.5) (width 1.016) (layer "B.Cu") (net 7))
 (segment (start 159.4668 121) (end 161 119.4668) (width 1.016) (layer "B.Cu") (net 7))
 (segment (start 100.0324 102.7176) (end 100 102.75) (width 1.016) (layer "B.Cu") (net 7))
 (segment (start 81 106.5) (end 91.5 106.5) (width 1.016) (layer "B.Cu") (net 7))
 (segment (start 82.5 115.5) (end 80 115.5) (width 1.016) (layer "B.Cu") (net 7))
 (segment (start 124.968 116.2812) (end 126 117.3132) (width 1.016) (layer "B.Cu") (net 7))
 (segment (start 79.5528 102.7176) (end 75.0609 107.2095) (width 1.016) (layer "B.Cu") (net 7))
 (segment (start 147.9296 113.5888) (end 114.562222 113.5888) (width 1.016) (layer "B.Cu") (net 7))
 (segment (start 152.5 118.1592) (end 147.9296 113.5888) (width 1.016) (layer "B.Cu") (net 7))
 (segment (start 83 122) (end 83 116) (width 1.016) (layer "B.Cu") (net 7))
 (segment (start 150 129.5804) (end 148 129.5804) (width 1.016) (layer "B.Cu") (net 7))
 (segment (start 118.9736 116.2812) (end 124.968 116.2812) (width 1.016) (layer "B.Cu") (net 7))
 (segment (start 140 122.5804) (end 142.4324 122.5804) (width 1.016) (layer "B.Cu") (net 7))
 (segment (start 62.85 107.23) (end 67.27 107.23) (width 1.016) (layer "B.Cu") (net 7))
 (segment (start 62.85 112.31) (end 75.19 112.31) (width 1.016) (layer "B.Cu") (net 7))
 (segment (start 147 128.5804) (end 145 128.5804) (width 1.016) (layer "B.Cu") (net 7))
 (segment (start 75.0609 107.2095) (end 73.4568 107.2095) (width 1.016) (layer "B.Cu") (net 7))
 (segment (start 54 109) (end 54 118.5) (width 1.016) (layer "B.Cu") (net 2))
 (segment (start 54 118.5) (end 50 118.5) (width 1.016) (layer "B.Cu") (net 2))
 (segment (start 60.31 107.23) (end 55.77 107.23) (width 1.016) (layer "B.Cu") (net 2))
 (segment (start 55.77 107.23) (end 54 109) (width 1.016) (layer "B.Cu") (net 2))
 (segment (start 58.23 109.77) (end 57.5 110.5) (width 1.016) (layer "B.Cu") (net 4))
 (segment (start 89.5 115.7636) (end 89.5 118.5) (width 1.016) (layer "B.Cu") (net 4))
 (segment (start 76.5 116.5) (end 79.2588 113.7412) (width 1.016) (layer "B.Cu") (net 4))
 (segment (start 79.2588 113.7412) (end 87.4776 113.7412) (width 1.016) (layer "B.Cu") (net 4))
 (segment (start 87.4776 113.7412) (end 89.5 115.7636) (width 1.016) (layer "B.Cu") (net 4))
 (segment (start 58.5 116.5) (end 76.5 116.5) (width 1.016) (layer "B.Cu") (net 4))
 (segment (start 60.31 109.77) (end 58.23 109.77) (width 1.016) (layer "B.Cu") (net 4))
 (segment (start 57.5 110.5) (end 57.5 115.5) (width 1.016) (layer "B.Cu") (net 4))
 (segment (start 57.5 115.5) (end 58.5 116.5) (width 1.016) (layer "B.Cu") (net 4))
 (segment (start 89.5 118.5) (end 85 118.5) (width 1.016) (layer "B.Cu") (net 4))
 (segment (start 60.31 114.31) (end 60.5 114.5) (width 1.016) (layer "B.Cu") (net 6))
 (segment (start 60.5 114.5) (end 75.5 114.5) (width 1.016) (layer "B.Cu") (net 6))
 (segment (start 75.5 114.5) (end 78.1384 111.8616) (width 1.016) (layer "B.Cu") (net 6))
 (segment (start 99.8616 111.8616) (end 111 123) (width 1.016) (layer "B.Cu") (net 6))
 (segment (start 120 120.9952) (end 120 118.5) (width 1.016) (layer "B.Cu") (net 6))
 (segment (start 124 118.5) (end 120 118.5) (width 1.016) (layer "B.Cu") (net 6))
 (segment (start 111 123) (end 117.9952 123) (width 1.016) (layer "B.Cu") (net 6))
 (segment (start 60.31 112.31) (end 60.31 114.31) (width 1.016) (layer "B.Cu") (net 6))
 (segment (start 78.1384 111.8616) (end 99.8616 111.8616) (width 1.016) (layer "B.Cu") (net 6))
 (segment (start 117.9952 123) (end 120 120.9952) (width 1.016) (layer "B.Cu") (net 6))
 (segment (start 155 118.5) (end 159 118.5) (width 1.016) (layer "B.Cu") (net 5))
 (segment (start 115.316 112.1664) (end 148.6664 112.1664) (width 1.016) (layer "B.Cu") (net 5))
 (segment (start 104.14 100.9904) (end 115.316 112.1664) (width 1.016) (layer "B.Cu") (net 5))
 (segment (start 66.5 101.04) (end 66.5 101) (width 1.016) (layer "B.Cu") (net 5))
 (segment (start 148.6664 112.1664) (end 155 118.5) (width 1.016) (layer "B.Cu") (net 5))
 (segment (start 66.5096 100.9904) (end 104.14 100.9904) (width 1.016) (layer "B.Cu") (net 5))
 (segment (start 62.85 104.69) (end 66.5 101.04) (width 1.016) (layer "B.Cu") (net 5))
 (segment (start 66.5 101) (end 66.5096 100.9904) (width 1.016) (layer "B.Cu") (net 5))
 (segment (start 91.5 104.5) (end 97.5 104.5) (width 1.016) (layer "B.Cu") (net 3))
 (segment (start 74.98 109.77) (end 80.25 104.5) (width 1.016) (layer "B.Cu") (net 3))
 (segment (start 62.85 109.77) (end 74.98 109.77) (width 1.016) (layer "B.Cu") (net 3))
 (segment (start 80.25 104.5) (end 91.5 104.5) (width 1.016) (layer "B.Cu") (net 3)))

